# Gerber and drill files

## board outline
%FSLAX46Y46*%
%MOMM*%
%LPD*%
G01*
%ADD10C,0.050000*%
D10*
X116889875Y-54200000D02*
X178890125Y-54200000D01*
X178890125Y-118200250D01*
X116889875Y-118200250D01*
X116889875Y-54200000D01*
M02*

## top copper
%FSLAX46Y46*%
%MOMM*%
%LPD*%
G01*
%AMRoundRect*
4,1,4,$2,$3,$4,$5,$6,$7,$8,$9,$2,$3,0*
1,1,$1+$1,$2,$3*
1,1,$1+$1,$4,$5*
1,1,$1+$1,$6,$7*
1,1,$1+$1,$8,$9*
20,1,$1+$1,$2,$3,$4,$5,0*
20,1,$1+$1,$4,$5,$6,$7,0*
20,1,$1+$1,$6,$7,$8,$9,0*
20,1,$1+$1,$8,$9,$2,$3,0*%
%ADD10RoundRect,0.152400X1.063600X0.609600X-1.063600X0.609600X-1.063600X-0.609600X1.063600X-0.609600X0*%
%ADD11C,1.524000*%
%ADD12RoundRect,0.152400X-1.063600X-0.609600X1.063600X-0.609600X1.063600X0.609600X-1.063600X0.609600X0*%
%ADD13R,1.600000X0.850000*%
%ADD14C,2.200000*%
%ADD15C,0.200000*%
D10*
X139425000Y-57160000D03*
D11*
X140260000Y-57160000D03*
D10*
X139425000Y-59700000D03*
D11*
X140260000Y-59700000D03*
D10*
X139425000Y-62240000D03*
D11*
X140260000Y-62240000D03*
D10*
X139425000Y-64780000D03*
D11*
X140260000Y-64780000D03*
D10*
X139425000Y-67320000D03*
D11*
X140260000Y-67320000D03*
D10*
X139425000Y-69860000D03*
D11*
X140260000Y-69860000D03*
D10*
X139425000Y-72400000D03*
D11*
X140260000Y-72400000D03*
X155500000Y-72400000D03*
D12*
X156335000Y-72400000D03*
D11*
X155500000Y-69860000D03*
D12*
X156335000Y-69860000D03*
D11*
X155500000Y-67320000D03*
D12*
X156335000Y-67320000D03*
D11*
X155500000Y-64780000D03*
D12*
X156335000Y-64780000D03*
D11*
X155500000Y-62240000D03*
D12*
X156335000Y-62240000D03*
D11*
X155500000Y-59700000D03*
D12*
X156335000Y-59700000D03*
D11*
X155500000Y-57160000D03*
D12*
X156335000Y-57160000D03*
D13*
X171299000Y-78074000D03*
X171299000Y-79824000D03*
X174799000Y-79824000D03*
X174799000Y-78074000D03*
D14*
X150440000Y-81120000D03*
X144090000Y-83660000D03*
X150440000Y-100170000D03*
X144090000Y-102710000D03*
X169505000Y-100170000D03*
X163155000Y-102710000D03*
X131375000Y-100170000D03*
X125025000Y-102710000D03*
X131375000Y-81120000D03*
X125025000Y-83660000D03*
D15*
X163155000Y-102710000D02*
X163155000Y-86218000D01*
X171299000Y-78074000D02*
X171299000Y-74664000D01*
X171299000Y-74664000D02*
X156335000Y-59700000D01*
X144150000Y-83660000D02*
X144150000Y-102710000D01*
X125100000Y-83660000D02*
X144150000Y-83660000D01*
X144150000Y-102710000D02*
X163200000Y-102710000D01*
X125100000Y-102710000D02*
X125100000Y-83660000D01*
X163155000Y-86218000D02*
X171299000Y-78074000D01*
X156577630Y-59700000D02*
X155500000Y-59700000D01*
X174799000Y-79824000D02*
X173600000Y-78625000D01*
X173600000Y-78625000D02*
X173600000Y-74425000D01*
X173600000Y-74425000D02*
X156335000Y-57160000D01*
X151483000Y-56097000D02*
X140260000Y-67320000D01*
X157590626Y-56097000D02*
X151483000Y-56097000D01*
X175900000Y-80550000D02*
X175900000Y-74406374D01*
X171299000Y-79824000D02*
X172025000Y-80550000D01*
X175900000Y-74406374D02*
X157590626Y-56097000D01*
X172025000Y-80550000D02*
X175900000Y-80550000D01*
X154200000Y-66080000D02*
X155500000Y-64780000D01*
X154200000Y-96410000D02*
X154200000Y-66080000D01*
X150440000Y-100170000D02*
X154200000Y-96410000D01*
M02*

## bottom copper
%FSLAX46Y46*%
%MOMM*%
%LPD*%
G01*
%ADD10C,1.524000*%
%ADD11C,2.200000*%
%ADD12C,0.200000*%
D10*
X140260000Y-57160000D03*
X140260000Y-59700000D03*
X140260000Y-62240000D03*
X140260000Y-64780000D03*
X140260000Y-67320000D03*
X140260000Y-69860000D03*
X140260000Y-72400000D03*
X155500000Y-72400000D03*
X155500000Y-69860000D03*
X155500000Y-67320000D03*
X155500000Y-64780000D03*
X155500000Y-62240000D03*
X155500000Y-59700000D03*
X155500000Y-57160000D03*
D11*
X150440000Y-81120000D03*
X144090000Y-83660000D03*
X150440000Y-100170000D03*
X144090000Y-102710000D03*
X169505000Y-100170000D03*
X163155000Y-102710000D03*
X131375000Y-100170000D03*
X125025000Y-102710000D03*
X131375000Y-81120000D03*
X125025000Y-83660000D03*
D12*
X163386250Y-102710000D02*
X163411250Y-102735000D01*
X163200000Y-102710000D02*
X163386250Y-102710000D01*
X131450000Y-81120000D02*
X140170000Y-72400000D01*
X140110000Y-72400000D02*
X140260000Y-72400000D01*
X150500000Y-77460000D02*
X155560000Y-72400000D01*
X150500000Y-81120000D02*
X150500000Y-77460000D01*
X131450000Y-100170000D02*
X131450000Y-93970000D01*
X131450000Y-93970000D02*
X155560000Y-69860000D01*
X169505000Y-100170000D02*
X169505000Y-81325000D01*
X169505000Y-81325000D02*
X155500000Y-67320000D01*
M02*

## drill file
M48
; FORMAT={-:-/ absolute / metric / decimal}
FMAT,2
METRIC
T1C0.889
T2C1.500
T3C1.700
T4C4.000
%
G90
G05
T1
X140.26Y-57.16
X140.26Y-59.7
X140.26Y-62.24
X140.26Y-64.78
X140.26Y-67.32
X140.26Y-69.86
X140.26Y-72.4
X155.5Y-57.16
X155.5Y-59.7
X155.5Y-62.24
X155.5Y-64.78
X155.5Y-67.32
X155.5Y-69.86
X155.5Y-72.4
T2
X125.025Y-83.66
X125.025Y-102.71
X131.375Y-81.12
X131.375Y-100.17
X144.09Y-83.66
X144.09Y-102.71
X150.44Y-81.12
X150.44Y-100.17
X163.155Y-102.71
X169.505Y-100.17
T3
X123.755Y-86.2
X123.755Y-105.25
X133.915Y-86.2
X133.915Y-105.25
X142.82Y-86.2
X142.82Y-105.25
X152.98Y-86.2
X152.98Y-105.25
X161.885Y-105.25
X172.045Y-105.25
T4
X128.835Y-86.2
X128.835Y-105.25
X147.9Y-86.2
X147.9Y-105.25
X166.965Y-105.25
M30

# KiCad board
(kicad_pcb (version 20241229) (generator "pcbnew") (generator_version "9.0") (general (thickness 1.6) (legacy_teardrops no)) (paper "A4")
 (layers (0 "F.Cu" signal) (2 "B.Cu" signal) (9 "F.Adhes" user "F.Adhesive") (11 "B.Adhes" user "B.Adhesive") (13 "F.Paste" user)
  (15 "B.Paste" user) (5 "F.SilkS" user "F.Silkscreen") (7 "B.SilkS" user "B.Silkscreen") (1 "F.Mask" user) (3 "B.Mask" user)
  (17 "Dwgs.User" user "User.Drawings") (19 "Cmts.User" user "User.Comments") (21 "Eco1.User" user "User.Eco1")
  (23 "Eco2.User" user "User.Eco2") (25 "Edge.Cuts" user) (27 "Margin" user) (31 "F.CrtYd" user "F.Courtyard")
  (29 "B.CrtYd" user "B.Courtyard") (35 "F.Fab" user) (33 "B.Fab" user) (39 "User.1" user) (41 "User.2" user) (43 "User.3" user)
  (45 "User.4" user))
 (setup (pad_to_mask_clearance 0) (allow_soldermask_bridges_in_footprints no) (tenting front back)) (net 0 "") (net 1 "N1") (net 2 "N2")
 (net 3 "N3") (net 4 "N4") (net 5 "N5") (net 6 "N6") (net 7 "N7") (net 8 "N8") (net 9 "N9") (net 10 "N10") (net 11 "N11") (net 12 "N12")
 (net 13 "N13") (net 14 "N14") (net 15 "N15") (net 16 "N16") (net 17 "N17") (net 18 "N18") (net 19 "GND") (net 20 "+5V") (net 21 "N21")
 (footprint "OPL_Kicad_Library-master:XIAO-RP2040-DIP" (layer "F.Cu") (at 147.88 64.78)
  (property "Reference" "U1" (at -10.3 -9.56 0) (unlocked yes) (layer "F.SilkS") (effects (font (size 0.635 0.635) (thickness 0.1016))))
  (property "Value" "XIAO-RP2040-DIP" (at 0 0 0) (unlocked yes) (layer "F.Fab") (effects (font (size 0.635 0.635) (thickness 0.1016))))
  (pad "1" smd roundrect (at -8.455 -7.62 180) (size 2.432 1.524) (layers "F.Cu" "F.Mask") (roundrect_rratio 0.1) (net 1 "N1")
   (thermal_bridge_angle 45))
  (pad "1" thru_hole circle (at -7.62 -7.62 180) (size 1.524 1.524) (drill 0.889) (layers "*.Cu" "*.Mask") (remove_unused_layers no)
   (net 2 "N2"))
  (pad "2" smd roundrect (at -8.455 -5.08 180) (size 2.432 1.524) (layers "F.Cu" "F.Mask") (roundrect_rratio 0.1) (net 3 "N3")
   (thermal_bridge_angle 45))
  (pad "2" thru_hole circle (at -7.62 -5.08 180) (size 1.524 1.524) (drill 0.889) (layers "*.Cu" "*.Mask") (remove_unused_layers no)
   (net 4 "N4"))
  (pad "3" smd roundrect (at -8.455 -2.54 180) (size 2.432 1.524) (layers "F.Cu" "F.Mask") (roundrect_rratio 0.1) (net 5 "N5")
   (thermal_bridge_angle 45))
  (pad "3" thru_hole circle (at -7.62 -2.54 180) (size 1.524 1.524) (drill 0.889) (layers "*.Cu" "*.Mask") (remove_unused_layers no)
   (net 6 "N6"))
  (pad "4" smd roundrect (at -8.455 0 180) (size 2.432 1.524) (layers "F.Cu" "F.Mask") (roundrect_rratio 0.1) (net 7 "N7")
   (thermal_bridge_angle 45))
  (pad "4" thru_hole circle (at -7.62 0 180) (size 1.524 1.524) (drill 0.889) (layers "*.Cu" "*.Mask") (remove_unused_layers no)
   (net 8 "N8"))
  (pad "5" smd roundrect (at -8.455 2.54 180) (size 2.432 1.524) (layers "F.Cu" "F.Mask") (roundrect_rratio 0.1) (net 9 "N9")
   (thermal_bridge_angle 45))
  (pad "5" thru_hole circle (at -7.62 2.54 180) (size 1.524 1.524) (drill 0.889) (layers "*.Cu" "*.Mask") (remove_unused_layers no)
   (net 9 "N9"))
  (pad "6" smd roundrect (at -8.455 5.08 180) (size 2.432 1.524) (layers "F.Cu" "F.Mask") (roundrect_rratio 0.1) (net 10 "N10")
   (thermal_bridge_angle 45))
  (pad "6" thru_hole circle (at -7.62 5.08 180) (size 1.524 1.524) (drill 0.889) (layers "*.Cu" "*.Mask") (remove_unused_layers no)
   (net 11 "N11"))
  (pad "7" smd roundrect (at -8.455 7.62 180) (size 2.432 1.524) (layers "F.Cu" "F.Mask") (roundrect_rratio 0.1) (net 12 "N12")
   (thermal_bridge_angle 45))
  (pad "7" thru_hole circle (at -7.62 7.62 180) (size 1.524 1.524) (drill 0.889) (layers "*.Cu" "*.Mask") (remove_unused_layers no)
   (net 12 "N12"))
  (pad "8" thru_hole circle (at 7.62 7.62) (size 1.524 1.524) (drill 0.889) (layers "*.Cu" "*.Mask") (remove_unused_layers no)
   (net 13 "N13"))
  (pad "8" smd roundrect (at 8.455 7.62) (size 2.432 1.524) (layers "F.Cu" "F.Mask") (roundrect_rratio 0.1) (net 13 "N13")
   (thermal_bridge_angle 45))
  (pad "9" thru_hole circle (at 7.62 5.08) (size 1.524 1.524) (drill 0.889) (layers "*.Cu" "*.Mask") (remove_unused_layers no)
   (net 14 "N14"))
  (pad "9" smd roundrect (at 8.455 5.08) (size 2.432 1.524) (layers "F.Cu" "F.Mask") (roundrect_rratio 0.1) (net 14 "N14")
   (thermal_bridge_angle 45))
  (pad "10" thru_hole circle (at 7.62 2.54) (size 1.524 1.524) (drill 0.889) (layers "*.Cu" "*.Mask") (remove_unused_layers no)
   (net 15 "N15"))
  (pad "10" smd roundrect (at 8.455 2.54) (size 2.432 1.524) (layers "F.Cu" "F.Mask") (roundrect_rratio 0.1) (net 15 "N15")
   (thermal_bridge_angle 45))
  (pad "11" thru_hole circle (at 7.62 0) (size 1.524 1.524) (drill 0.889) (layers "*.Cu" "*.Mask") (remove_unused_layers no) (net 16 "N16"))
  (pad "11" smd roundrect (at 8.455 0) (size 2.432 1.524) (layers "F.Cu" "F.Mask") (roundrect_rratio 0.1) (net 16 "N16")
   (thermal_bridge_angle 45))
  (pad "12" thru_hole circle (at 7.62 -2.54) (size 1.524 1.524) (drill 0.889) (layers "*.Cu" "*.Mask") (remove_unused_layers no)
   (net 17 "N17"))
  (pad "12" smd roundrect (at 8.455 -2.54) (size 2.432 1.524) (layers "F.Cu" "F.Mask") (roundrect_rratio 0.1) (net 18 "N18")
   (thermal_bridge_angle 45))
  (pad "13" thru_hole circle (at 7.62 -5.08) (size 1.524 1.524) (drill 0.889) (layers "*.Cu" "*.Mask") (remove_unused_layers no)
   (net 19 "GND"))
  (pad "13" smd roundrect (at 8.455 -5.08) (size 2.432 1.524) (layers "F.Cu" "F.Mask") (roundrect_rratio 0.1) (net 19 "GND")
   (thermal_bridge_angle 45))
  (pad "14" thru_hole circle (at 7.62 -7.62) (size 1.524 1.524) (drill 0.889) (layers "*.Cu" "*.Mask") (remove_unused_layers no)
   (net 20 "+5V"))
  (pad "14" smd roundrect (at 8.455 -7.62) (size 2.432 1.524) (layers "F.Cu" "F.Mask") (roundrect_rratio 0.1) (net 20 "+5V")
   (thermal_bridge_angle 45)))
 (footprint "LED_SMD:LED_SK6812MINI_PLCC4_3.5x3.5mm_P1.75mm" (layer "F.Cu") (at 173.049 78.949)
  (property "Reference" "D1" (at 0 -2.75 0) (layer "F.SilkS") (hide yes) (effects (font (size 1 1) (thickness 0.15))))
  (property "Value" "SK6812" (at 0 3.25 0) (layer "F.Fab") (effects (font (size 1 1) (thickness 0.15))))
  (pad "1" smd rect (at -1.75 -0.875) (size 1.6 0.85) (layers "F.Cu" "F.Mask" "F.Paste") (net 19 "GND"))
  (pad "2" smd rect (at -1.75 0.875) (size 1.6 0.85) (layers "F.Cu" "F.Mask" "F.Paste") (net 9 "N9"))
  (pad "3" smd rect (at 1.75 0.875) (size 1.6 0.85) (layers "F.Cu" "F.Mask" "F.Paste") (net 20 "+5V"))
  (pad "4" smd rect (at 1.75 -0.875) (size 1.6 0.85) (layers "F.Cu" "F.Mask" "F.Paste") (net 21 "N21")))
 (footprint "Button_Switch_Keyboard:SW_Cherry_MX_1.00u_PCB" (layer "F.Cu") (at 150.44 81.12)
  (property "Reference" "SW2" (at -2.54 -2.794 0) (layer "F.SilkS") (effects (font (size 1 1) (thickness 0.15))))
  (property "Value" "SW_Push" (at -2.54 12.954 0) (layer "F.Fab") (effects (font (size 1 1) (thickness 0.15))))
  (pad "" np_thru_hole circle (at -7.62 5.08) (size 1.7 1.7) (drill 1.7) (layers "*.Cu" "*.Mask"))
  (pad "" np_thru_hole circle (at -2.54 5.08) (size 4 4) (drill 4) (layers "*.Cu" "*.Mask"))
  (pad "" np_thru_hole circle (at 2.54 5.08) (size 1.7 1.7) (drill 1.7) (layers "*.Cu" "*.Mask"))
  (pad "1" thru_hole circle (at 0 0) (size 2.2 2.2) (drill 1.5) (layers "*.Cu" "*.Mask") (remove_unused_layers no) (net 13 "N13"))
  (pad "2" thru_hole circle (at -6.35 2.54) (size 2.2 2.2) (drill 1.5) (layers "*.Cu" "*.Mask") (remove_unused_layers no) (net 19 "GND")))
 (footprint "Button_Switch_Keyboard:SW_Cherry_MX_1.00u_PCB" (layer "F.Cu") (at 150.44 100.17)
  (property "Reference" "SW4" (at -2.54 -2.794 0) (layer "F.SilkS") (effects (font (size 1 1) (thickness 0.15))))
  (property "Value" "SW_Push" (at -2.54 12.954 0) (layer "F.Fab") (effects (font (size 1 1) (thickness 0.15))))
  (pad "" np_thru_hole circle (at -7.62 5.08) (size 1.7 1.7) (drill 1.7) (layers "*.Cu" "*.Mask"))
  (pad "" np_thru_hole circle (at -2.54 5.08) (size 4 4) (drill 4) (layers "*.Cu" "*.Mask"))
  (pad "" np_thru_hole circle (at 2.54 5.08) (size 1.7 1.7) (drill 1.7) (layers "*.Cu" "*.Mask"))
  (pad "1" thru_hole circle (at 0 0) (size 2.2 2.2) (drill 1.5) (layers "*.Cu" "*.Mask") (remove_unused_layers no) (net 16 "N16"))
  (pad "2" thru_hole circle (at -6.35 2.54) (size 2.2 2.2) (drill 1.5) (layers "*.Cu" "*.Mask") (remove_unused_layers no) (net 19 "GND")))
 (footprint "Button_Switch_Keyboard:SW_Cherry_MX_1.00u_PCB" (layer "F.Cu") (at 169.505 100.17)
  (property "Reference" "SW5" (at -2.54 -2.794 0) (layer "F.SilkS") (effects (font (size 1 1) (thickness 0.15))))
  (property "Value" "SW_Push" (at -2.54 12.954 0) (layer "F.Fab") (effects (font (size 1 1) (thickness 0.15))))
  (pad "" np_thru_hole circle (at -7.62 5.08) (size 1.7 1.7) (drill 1.7) (layers "*.Cu" "*.Mask"))
  (pad "" np_thru_hole circle (at -2.54 5.08) (size 4 4) (drill 4) (layers "*.Cu" "*.Mask"))
  (pad "" np_thru_hole circle (at 2.54 5.08) (size 1.7 1.7) (drill 1.7) (layers "*.Cu" "*.Mask"))
  (pad "1" thru_hole circle (at 0 0) (size 2.2 2.2) (drill 1.5) (layers "*.Cu" "*.Mask") (remove_unused_layers no) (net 15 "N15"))
  (pad "2" thru_hole circle (at -6.35 2.54) (size 2.2 2.2) (drill 1.5) (layers "*.Cu" "*.Mask") (remove_unused_layers no) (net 19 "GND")))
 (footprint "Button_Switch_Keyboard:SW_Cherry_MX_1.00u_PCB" (layer "F.Cu") (at 131.375 100.17)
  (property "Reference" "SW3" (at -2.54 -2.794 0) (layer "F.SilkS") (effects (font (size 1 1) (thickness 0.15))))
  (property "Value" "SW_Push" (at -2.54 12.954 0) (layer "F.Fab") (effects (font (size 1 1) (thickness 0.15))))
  (pad "" np_thru_hole circle (at -7.62 5.08) (size 1.7 1.7) (drill 1.7) (layers "*.Cu" "*.Mask"))
  (pad "" np_thru_hole circle (at -2.54 5.08) (size 4 4) (drill 4) (layers "*.Cu" "*.Mask"))
  (pad "" np_thru_hole circle (at 2.54 5.08) (size 1.7 1.7) (drill 1.7) (layers "*.Cu" "*.Mask"))
  (pad "1" thru_hole circle (at 0 0) (size 2.2 2.2) (drill 1.5) (layers "*.Cu" "*.Mask") (remove_unused_layers no) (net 14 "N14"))
  (pad "2" thru_hole circle (at -6.35 2.54) (size 2.2 2.2) (drill 1.5) (layers "*.Cu" "*.Mask") (remove_unused_layers no) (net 19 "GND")))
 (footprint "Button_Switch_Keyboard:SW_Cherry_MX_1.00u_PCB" (layer "F.Cu") (at 131.375 81.12)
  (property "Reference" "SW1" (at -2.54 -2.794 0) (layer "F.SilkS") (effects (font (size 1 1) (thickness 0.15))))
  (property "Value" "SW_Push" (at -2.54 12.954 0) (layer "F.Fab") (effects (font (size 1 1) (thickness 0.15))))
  (pad "" np_thru_hole circle (at -7.62 5.08) (size 1.7 1.7) (drill 1.7) (layers "*.Cu" "*.Mask"))
  (pad "" np_thru_hole circle (at -2.54 5.08) (size 4 4) (drill 4) (layers "*.Cu" "*.Mask"))
  (pad "" np_thru_hole circle (at 2.54 5.08) (size 1.7 1.7) (drill 1.7) (layers "*.Cu" "*.Mask"))
  (pad "1" thru_hole circle (at 0 0) (size 2.2 2.2) (drill 1.5) (layers "*.Cu" "*.Mask") (remove_unused_layers no) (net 12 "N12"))
  (pad "2" thru_hole circle (at -6.35 2.54) (size 2.2 2.2) (drill 1.5) (layers "*.Cu" "*.Mask") (remove_unused_layers no) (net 19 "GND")))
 (gr_rect (start 116.889875 54.2) (end 178.890125 118.20025) (stroke (width 0.05) (type default)) (fill no) (layer "Edge.Cuts"))
 (segment (start 163.155 102.71) (end 163.155 86.218) (width 0.2) (layer "F.Cu") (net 19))
 (segment (start 171.299 78.074) (end 171.299 74.664) (width 0.2) (layer "F.Cu") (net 19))
 (segment (start 171.299 74.664) (end 156.335 59.7) (width 0.2) (layer "F.Cu") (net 19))
 (segment (start 144.15 83.66) (end 144.15 102.71) (width 0.2) (layer "F.Cu") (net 19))
 (segment (start 125.1 83.66) (end 144.15 83.66) (width 0.2) (layer "F.Cu") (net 19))
 (segment (start 144.15 102.71) (end 163.2 102.71) (width 0.2) (layer "F.Cu") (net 19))
 (segment (start 125.1 102.71) (end 125.1 83.66) (width 0.2) (layer "F.Cu") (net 19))
 (segment (start 163.155 86.218) (end 171.299 78.074) (width 0.2) (layer "F.Cu") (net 19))
 (segment (start 156.57763 59.7) (end 155.5 59.7) (width 0.2) (layer "F.Cu") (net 19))
 (segment (start 163.38625 102.71) (end 163.41125 102.735) (width 0.2) (layer "B.Cu") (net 19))
 (segment (start 163.2 102.71) (end 163.38625 102.71) (width 0.2) (layer "B.Cu") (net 19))
 (segment (start 174.799 79.824) (end 173.6 78.625) (width 0.2) (layer "F.Cu") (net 20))
 (segment (start 173.6 78.625) (end 173.6 74.425) (width 0.2) (layer "F.Cu") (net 20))
 (segment (start 173.6 74.425) (end 156.335 57.16) (width 0.2) (layer "F.Cu") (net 20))
 (segment (start 151.483 56.097) (end 140.26 67.32) (width 0.2) (layer "F.Cu") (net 9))
 (segment (start 157.590626 56.097) (end 151.483 56.097) (width 0.2) (layer "F.Cu") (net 9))
 (segment (start 175.9 80.55) (end 175.9 74.406374) (width 0.2) (layer "F.Cu") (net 9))
 (segment (start 171.299 79.824) (end 172.025 80.55) (width 0.2) (layer "F.Cu") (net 9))
 (segment (start 175.9 74.406374) (end 157.590626 56.097) (width 0.2) (layer "F.Cu") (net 9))
 (segment (start 172.025 80.55) (end 175.9 80.55) (width 0.2) (layer "F.Cu") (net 9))
 (segment (start 131.45 81.12) (end 140.17 72.4) (width 0.2) (layer "B.Cu") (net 12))
 (segment (start 140.11 72.4) (end 140.26 72.4) (width 0.2) (layer "B.Cu") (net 12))
 (segment (start 150.5 77.46) (end 155.56 72.4) (width 0.2) (layer "B.Cu") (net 13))
 (segment (start 150.5 81.12) (end 150.5 77.46) (width 0.2) (layer "B.Cu") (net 13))
 (segment (start 131.45 100.17) (end 131.45 93.97) (width 0.2) (layer "B.Cu") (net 14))
 (segment (start 131.45 93.97) (end 155.56 69.86) (width 0.2) (layer "B.Cu") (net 14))
 (segment (start 154.2 66.08) (end 155.5 64.78) (width 0.2) (layer "F.Cu") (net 16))
 (segment (start 154.2 96.41) (end 154.2 66.08) (width 0.2) (layer "F.Cu") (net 16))
 (segment (start 150.44 100.17) (end 154.2 96.41) (width 0.2) (layer "F.Cu") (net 16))
 (segment (start 169.505 100.17) (end 169.505 81.325) (width 0.2) (layer "B.Cu") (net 15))
 (segment (start 169.505 81.325) (end 155.5 67.32) (width 0.2) (layer "B.Cu") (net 15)))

